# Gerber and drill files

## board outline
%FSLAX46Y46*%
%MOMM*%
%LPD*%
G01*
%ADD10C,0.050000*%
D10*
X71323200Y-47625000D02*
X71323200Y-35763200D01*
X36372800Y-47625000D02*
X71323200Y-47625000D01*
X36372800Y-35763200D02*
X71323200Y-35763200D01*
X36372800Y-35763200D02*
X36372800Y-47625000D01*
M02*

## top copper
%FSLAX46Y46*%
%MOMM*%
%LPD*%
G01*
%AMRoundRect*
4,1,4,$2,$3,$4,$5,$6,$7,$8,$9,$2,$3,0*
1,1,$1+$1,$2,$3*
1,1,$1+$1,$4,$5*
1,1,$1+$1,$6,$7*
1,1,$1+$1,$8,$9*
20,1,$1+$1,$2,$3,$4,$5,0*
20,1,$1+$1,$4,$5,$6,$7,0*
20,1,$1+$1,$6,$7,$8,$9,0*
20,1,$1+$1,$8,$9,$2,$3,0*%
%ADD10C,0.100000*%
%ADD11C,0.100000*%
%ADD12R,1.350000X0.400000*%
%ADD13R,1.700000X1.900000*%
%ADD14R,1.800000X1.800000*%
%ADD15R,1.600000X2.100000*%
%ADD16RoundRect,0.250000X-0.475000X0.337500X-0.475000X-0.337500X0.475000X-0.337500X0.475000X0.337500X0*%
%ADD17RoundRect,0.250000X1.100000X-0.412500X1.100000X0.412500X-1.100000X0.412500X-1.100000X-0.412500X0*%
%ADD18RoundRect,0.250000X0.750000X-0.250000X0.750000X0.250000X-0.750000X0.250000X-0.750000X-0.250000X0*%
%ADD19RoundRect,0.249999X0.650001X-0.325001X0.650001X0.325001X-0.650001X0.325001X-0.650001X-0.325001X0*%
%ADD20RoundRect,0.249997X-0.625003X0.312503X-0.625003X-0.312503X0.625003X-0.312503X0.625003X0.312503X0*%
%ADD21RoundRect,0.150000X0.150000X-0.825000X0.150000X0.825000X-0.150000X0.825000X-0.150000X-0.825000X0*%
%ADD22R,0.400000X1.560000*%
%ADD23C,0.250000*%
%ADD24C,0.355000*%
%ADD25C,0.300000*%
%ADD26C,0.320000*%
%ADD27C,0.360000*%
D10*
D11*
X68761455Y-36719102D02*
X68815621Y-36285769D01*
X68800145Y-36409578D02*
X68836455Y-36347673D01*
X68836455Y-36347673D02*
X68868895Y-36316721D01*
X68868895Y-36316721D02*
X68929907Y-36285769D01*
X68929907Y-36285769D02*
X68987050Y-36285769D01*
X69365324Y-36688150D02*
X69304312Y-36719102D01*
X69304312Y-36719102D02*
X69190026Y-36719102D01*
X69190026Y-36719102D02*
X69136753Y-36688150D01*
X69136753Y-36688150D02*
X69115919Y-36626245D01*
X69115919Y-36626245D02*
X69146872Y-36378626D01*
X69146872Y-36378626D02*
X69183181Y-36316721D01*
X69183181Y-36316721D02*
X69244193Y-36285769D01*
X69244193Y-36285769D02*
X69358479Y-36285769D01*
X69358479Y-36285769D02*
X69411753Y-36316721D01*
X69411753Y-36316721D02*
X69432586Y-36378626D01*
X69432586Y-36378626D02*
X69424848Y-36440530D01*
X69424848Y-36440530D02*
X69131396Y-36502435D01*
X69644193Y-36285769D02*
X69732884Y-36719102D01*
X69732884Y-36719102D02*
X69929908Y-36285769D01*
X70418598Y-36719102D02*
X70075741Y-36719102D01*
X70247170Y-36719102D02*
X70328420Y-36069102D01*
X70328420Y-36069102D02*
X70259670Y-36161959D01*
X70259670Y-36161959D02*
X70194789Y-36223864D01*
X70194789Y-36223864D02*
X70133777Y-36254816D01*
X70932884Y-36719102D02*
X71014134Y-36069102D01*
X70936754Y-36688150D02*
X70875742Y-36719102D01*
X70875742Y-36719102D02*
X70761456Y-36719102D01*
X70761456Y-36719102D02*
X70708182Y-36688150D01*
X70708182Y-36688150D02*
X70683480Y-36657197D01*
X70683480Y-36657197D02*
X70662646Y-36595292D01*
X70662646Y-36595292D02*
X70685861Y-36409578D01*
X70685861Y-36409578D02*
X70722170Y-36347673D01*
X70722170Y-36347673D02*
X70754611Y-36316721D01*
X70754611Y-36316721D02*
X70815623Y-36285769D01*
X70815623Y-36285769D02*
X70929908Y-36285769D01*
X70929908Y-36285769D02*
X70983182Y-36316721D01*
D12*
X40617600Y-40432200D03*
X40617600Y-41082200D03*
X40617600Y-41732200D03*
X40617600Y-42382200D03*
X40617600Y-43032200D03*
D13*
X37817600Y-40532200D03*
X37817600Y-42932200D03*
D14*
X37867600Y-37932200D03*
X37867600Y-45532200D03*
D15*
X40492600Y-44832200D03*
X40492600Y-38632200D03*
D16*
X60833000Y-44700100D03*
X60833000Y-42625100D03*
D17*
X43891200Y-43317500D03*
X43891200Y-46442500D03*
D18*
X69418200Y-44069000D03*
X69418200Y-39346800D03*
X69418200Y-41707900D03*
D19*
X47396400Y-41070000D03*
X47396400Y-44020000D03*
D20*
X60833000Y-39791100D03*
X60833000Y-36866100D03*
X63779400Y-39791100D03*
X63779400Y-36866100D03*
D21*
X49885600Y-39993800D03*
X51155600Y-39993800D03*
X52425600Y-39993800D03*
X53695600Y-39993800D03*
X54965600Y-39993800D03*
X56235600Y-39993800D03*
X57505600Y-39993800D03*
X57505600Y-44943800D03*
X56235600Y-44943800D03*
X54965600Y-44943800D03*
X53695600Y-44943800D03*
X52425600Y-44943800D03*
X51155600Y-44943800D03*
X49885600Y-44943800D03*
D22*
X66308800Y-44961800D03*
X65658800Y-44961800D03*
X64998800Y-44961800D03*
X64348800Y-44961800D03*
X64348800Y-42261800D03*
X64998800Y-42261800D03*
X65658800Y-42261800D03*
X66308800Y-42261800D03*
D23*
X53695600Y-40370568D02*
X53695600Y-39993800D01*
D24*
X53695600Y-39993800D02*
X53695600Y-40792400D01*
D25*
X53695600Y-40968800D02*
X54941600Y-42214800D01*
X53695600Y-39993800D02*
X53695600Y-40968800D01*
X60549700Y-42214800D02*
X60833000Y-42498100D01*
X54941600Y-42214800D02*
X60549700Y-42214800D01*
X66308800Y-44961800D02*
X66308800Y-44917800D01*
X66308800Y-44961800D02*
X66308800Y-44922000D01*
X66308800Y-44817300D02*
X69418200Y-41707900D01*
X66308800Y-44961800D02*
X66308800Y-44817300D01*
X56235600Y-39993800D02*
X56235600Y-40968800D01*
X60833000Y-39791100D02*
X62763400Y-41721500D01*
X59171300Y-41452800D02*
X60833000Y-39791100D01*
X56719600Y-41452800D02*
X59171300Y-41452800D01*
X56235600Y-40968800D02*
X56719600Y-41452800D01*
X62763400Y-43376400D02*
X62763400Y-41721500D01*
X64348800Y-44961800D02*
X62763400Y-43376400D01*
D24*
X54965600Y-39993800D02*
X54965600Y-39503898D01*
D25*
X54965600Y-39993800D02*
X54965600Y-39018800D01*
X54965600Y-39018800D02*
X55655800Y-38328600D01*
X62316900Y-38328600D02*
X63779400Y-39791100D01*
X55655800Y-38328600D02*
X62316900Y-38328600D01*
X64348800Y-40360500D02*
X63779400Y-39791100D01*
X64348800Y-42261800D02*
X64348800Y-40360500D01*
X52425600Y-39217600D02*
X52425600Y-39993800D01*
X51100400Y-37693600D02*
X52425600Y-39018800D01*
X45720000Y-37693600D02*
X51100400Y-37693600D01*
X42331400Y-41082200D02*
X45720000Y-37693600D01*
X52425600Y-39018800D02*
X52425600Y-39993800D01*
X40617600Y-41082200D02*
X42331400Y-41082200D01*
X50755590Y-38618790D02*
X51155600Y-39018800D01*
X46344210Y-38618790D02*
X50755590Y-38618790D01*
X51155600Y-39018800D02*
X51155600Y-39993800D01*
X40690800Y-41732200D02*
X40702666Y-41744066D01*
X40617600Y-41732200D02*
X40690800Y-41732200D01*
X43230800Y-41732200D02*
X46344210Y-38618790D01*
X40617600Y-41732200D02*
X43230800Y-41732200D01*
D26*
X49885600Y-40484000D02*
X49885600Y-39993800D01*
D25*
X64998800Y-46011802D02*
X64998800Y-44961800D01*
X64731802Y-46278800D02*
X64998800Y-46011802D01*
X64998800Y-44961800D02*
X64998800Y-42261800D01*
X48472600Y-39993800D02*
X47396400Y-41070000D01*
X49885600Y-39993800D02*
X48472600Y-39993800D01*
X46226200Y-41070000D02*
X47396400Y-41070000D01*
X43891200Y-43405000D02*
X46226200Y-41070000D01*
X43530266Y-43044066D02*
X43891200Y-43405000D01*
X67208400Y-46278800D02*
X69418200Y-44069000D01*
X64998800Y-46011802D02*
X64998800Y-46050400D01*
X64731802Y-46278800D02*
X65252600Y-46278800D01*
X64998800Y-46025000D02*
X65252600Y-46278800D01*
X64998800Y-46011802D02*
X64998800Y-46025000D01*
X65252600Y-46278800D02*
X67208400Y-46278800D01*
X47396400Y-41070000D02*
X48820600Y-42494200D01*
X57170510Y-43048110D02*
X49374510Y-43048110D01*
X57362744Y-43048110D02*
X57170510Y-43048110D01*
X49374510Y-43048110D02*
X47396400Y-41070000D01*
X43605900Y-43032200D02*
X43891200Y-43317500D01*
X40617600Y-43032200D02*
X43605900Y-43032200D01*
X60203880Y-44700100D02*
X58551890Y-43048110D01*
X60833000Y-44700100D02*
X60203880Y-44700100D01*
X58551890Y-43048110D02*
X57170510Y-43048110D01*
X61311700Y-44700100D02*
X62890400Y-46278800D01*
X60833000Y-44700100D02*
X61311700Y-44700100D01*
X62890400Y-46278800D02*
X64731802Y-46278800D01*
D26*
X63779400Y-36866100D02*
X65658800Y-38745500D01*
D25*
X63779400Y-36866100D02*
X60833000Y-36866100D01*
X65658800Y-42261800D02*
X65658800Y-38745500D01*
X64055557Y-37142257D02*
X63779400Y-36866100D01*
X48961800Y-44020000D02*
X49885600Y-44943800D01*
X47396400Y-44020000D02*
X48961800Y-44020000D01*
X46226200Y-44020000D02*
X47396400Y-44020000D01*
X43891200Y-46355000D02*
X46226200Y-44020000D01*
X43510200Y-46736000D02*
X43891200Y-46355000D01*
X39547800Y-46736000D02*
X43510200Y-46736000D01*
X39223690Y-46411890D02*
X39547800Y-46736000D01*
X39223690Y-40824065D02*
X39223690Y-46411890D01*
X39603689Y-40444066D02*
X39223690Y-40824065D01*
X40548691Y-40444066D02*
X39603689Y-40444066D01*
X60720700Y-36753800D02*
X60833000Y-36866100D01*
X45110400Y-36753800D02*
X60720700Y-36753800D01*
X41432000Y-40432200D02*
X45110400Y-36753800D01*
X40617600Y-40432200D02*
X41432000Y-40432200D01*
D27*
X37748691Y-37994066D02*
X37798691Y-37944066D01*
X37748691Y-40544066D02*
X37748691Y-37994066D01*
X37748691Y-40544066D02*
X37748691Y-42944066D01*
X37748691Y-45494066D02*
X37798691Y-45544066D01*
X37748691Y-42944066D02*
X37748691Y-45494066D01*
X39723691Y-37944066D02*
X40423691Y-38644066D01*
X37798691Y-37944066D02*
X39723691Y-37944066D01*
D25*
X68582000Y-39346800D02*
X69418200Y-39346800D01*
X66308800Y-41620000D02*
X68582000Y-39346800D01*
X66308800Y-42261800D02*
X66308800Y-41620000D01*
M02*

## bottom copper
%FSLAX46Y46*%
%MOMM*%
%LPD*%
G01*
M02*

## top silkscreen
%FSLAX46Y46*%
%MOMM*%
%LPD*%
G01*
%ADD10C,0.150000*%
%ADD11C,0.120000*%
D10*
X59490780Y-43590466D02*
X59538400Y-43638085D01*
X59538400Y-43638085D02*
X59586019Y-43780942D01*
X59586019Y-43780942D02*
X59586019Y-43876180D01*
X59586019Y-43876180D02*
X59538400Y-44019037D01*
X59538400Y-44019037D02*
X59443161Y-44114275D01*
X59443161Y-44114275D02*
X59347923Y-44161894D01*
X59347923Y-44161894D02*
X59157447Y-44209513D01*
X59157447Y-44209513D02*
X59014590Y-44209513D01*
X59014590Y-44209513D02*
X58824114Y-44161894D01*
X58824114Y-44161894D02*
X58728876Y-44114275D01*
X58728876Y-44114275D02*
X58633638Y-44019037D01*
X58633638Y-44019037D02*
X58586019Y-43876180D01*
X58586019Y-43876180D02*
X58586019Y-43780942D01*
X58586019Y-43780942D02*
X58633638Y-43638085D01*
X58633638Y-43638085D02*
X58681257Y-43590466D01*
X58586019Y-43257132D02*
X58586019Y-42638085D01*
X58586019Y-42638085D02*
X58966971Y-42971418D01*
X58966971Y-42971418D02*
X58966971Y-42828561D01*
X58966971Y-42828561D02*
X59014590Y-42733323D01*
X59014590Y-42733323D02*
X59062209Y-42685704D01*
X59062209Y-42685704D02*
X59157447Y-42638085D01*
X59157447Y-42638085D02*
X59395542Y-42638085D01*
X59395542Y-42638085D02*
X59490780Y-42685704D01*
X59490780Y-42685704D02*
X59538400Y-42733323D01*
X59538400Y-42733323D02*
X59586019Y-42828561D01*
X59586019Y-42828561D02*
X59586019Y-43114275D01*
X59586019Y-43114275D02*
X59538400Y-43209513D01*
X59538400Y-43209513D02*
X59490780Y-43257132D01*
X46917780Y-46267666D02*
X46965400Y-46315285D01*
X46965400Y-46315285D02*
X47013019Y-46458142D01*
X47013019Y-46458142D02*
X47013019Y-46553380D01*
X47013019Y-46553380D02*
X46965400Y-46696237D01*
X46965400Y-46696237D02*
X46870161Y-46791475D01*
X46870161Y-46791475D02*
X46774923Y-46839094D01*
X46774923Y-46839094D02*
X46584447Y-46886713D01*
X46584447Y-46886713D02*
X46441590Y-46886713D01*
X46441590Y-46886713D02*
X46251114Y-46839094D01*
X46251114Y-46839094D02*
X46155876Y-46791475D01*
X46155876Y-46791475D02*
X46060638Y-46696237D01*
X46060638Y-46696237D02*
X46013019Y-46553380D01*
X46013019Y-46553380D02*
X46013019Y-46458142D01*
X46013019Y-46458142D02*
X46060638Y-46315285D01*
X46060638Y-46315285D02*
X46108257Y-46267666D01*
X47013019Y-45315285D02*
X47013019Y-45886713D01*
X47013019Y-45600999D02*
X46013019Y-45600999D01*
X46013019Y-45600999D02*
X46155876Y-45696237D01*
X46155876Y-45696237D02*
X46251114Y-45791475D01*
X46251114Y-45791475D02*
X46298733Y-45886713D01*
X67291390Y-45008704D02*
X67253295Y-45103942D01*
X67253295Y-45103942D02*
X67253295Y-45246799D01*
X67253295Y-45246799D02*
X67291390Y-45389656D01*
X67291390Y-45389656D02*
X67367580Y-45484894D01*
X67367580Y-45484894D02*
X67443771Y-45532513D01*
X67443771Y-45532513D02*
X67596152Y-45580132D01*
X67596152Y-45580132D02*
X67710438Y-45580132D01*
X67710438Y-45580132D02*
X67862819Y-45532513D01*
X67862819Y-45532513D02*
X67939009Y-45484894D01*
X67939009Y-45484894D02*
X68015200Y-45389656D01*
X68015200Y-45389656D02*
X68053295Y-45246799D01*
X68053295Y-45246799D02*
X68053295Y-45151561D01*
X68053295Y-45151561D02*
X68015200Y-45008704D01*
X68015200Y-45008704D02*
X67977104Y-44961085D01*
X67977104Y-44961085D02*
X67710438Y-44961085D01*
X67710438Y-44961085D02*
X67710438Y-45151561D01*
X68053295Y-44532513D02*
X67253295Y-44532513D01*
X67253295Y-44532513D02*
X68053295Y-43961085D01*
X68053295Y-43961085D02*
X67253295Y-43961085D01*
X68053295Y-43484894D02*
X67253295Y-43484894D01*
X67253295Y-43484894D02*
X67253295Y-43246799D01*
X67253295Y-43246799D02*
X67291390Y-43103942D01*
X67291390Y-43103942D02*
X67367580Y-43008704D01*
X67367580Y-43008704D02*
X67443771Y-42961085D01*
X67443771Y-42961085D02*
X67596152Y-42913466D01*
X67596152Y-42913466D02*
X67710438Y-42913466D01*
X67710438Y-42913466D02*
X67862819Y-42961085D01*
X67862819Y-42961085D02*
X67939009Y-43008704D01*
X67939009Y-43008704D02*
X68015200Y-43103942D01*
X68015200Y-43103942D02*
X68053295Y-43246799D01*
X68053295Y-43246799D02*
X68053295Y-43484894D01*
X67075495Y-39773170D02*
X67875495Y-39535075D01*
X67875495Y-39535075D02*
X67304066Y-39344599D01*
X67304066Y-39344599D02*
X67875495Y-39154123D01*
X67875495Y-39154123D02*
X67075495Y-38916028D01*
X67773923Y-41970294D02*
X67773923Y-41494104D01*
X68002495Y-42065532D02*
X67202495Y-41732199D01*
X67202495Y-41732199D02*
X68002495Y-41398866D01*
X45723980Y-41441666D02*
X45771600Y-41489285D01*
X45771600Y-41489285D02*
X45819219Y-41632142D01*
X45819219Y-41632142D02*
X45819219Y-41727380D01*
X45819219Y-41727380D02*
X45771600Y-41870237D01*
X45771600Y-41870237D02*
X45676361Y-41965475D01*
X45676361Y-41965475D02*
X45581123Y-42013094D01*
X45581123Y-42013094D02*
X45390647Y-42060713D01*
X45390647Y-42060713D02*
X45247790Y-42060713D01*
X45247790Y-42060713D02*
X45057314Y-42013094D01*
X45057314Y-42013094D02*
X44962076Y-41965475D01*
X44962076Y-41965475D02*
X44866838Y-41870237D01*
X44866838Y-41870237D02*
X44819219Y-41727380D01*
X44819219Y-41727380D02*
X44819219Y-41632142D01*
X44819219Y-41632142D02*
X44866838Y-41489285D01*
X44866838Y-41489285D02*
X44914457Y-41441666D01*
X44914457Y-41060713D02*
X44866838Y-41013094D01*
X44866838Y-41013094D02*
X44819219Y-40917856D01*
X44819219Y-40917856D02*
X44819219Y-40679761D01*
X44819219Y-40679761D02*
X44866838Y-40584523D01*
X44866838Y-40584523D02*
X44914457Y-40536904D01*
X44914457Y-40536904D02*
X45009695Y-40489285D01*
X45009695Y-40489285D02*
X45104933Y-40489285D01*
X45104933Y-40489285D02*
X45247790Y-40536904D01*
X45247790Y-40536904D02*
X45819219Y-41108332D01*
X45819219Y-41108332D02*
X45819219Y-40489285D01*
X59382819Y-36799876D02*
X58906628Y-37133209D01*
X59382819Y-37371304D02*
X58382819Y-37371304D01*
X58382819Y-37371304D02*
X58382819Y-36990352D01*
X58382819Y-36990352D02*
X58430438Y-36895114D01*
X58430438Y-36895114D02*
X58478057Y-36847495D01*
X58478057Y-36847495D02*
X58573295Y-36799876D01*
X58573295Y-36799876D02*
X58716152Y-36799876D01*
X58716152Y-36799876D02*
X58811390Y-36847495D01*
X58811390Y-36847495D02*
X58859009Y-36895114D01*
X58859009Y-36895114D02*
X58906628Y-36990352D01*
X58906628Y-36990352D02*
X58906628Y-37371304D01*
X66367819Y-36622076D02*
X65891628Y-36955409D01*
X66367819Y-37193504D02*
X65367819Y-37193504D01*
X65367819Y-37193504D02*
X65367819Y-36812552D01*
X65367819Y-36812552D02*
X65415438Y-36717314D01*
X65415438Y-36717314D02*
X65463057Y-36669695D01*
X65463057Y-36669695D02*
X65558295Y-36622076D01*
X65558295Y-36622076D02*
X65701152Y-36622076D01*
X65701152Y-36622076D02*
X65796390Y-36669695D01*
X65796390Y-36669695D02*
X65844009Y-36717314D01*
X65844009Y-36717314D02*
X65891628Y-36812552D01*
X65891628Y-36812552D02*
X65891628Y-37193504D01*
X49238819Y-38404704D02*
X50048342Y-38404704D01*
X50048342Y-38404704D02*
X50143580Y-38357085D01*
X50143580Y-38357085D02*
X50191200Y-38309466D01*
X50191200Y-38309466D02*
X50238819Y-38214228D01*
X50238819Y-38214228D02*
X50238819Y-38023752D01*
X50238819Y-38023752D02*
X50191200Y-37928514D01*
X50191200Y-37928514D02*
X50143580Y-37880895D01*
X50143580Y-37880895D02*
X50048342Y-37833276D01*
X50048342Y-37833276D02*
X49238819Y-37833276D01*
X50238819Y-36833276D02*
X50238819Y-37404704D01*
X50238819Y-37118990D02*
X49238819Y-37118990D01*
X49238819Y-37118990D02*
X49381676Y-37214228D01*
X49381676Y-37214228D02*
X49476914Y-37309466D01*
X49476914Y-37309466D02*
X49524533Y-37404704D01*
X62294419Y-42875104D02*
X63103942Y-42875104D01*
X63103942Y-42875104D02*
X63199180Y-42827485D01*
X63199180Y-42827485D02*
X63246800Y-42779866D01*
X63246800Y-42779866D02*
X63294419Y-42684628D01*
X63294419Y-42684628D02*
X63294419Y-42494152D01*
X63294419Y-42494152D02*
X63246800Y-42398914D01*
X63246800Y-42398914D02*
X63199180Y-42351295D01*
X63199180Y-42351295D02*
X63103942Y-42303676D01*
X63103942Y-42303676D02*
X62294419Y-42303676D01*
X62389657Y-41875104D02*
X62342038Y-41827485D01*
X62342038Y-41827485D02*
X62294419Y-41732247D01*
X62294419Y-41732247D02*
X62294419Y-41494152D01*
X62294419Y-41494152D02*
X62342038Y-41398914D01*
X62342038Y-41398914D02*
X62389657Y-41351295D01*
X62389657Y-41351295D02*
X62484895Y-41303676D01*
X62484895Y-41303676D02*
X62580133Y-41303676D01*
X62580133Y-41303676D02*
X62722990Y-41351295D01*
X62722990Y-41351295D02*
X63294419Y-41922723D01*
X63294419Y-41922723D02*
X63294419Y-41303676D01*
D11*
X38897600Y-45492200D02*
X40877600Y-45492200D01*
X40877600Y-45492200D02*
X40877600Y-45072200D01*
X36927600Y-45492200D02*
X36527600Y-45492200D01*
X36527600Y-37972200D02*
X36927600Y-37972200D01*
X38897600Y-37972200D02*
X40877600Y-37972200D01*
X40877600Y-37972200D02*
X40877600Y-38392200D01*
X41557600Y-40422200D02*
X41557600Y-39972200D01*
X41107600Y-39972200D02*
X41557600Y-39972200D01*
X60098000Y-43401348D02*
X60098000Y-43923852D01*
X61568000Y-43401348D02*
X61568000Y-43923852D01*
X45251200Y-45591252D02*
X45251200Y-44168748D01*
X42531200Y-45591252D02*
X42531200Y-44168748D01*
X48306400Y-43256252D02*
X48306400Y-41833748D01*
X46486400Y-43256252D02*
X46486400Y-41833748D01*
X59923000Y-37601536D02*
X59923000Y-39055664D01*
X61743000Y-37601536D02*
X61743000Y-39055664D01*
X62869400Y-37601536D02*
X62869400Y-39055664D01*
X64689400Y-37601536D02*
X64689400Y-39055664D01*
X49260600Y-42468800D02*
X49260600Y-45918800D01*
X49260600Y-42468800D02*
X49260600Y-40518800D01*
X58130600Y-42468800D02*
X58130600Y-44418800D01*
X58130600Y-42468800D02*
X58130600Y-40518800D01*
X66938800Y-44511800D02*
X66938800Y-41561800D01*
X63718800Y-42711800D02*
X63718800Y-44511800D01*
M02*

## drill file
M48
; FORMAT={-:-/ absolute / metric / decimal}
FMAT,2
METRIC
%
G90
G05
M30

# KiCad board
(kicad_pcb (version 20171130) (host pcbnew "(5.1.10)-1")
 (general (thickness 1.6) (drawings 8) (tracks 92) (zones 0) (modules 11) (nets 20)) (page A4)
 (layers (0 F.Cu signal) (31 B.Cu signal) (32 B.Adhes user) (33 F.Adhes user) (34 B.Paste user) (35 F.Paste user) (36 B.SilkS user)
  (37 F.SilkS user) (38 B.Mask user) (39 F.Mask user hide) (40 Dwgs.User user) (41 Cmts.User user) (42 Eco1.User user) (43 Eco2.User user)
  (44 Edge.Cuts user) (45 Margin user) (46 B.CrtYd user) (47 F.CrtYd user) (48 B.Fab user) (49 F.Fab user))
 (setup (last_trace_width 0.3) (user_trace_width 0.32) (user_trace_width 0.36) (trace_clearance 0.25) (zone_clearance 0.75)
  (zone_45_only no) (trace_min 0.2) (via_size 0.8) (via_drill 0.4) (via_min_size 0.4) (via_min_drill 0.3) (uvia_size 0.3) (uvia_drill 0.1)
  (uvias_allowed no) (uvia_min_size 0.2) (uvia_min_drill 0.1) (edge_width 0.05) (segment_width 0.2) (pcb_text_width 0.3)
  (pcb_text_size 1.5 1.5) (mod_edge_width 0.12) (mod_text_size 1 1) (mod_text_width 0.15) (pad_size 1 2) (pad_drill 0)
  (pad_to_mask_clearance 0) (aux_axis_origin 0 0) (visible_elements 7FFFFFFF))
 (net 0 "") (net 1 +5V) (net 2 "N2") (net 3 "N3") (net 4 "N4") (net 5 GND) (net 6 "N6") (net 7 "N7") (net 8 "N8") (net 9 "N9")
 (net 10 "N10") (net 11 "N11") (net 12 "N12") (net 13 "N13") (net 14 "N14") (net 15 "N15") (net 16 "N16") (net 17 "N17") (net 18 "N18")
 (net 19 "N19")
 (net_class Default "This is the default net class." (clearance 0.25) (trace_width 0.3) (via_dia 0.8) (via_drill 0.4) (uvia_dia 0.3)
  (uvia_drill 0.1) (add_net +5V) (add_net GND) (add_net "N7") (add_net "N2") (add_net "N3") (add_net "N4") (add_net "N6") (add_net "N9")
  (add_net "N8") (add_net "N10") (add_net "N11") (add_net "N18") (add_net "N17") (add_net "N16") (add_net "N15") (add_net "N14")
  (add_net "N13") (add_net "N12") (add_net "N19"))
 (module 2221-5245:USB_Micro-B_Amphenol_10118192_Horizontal (layer F.Cu) (at 39.2176 41.7322 270)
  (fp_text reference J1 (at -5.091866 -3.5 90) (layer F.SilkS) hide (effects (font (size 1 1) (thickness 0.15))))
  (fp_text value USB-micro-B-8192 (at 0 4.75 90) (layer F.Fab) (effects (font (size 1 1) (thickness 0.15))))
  (fp_line (start 3.76 0.32) (end 3.76 -1.66) (layer F.SilkS) (width 0.12))
  (fp_line (start 3.76 -1.66) (end 3.34 -1.66) (layer F.SilkS) (width 0.12))
  (fp_line (start 3.76 2.29) (end 3.76 2.69) (layer F.SilkS) (width 0.12))
  (fp_line (start -3.76 2.69) (end -3.76 2.29) (layer F.SilkS) (width 0.12))
  (fp_line (start -3.76 0.32) (end -3.76 -1.66) (layer F.SilkS) (width 0.12))
  (fp_line (start -3.76 -1.66) (end -3.34 -1.66) (layer F.SilkS) (width 0.12))
  (fp_line (start -1.31 -2.34) (end -1.76 -2.34) (layer F.SilkS) (width 0.12))
  (fp_line (start -1.76 -1.89) (end -1.76 -2.34) (layer F.SilkS) (width 0.12))
  (pad 1 smd rect (at -1.3 -1.4 270) (size 0.4 1.35) (layers F.Cu F.Paste F.Mask) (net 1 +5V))
  (pad 2 smd rect (at -0.65 -1.4 270) (size 0.4 1.35) (layers F.Cu F.Paste F.Mask) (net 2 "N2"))
  (pad 3 smd rect (at 0 -1.4 270) (size 0.4 1.35) (layers F.Cu F.Paste F.Mask) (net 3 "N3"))
  (pad 4 smd rect (at 0.65 -1.4 270) (size 0.4 1.35) (layers F.Cu F.Paste) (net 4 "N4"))
  (pad 5 smd rect (at 1.3 -1.4 270) (size 0.4 1.35) (layers F.Cu F.Paste F.Mask) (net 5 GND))
  (pad 6 smd rect (at -1.2 1.4 270) (size 1.9 1.7) (layers F.Cu F.Paste F.Mask) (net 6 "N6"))
  (pad 6 smd rect (at 1.2 1.4 270) (size 1.9 1.7) (layers F.Cu F.Paste F.Mask) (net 6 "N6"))
  (pad 6 smd rect (at -3.8 1.35 270) (size 1.8 1.8) (layers F.Cu F.Paste F.Mask) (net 6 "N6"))
  (pad 6 smd rect (at 3.8 1.35 270) (size 1.8 1.8) (layers F.Cu F.Paste F.Mask) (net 6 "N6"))
  (pad 6 smd rect (at 3.1 -1.275 270) (size 2.1 1.6) (layers F.Cu F.Paste F.Mask) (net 6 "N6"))
  (pad 6 smd rect (at -3.1 -1.275 270) (size 2.1 1.6) (layers F.Cu F.Paste F.Mask) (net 6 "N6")))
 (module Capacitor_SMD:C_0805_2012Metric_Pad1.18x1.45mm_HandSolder (layer F.Cu) (at 60.833 43.6626 270)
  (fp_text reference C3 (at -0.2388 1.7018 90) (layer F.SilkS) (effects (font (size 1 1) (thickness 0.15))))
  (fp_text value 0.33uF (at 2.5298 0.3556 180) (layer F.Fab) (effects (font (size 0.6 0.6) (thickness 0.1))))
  (fp_line (start -0.261252 0.735) (end 0.261252 0.735) (layer F.SilkS) (width 0.12))
  (fp_line (start -0.261252 -0.735) (end 0.261252 -0.735) (layer F.SilkS) (width 0.12))
  (pad 2 smd roundrect (at 1.0375 0 270) (size 1.175 1.45) (layers F.Cu F.Paste F.Mask) (roundrect_rratio 0.212766) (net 5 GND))
  (pad 1 smd roundrect (at -1.0375 0 270) (size 1.175 1.45) (layers F.Cu F.Paste F.Mask) (roundrect_rratio 0.212766) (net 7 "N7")))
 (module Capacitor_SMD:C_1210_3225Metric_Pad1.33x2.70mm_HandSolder (layer F.Cu) (at 43.8912 44.88 90)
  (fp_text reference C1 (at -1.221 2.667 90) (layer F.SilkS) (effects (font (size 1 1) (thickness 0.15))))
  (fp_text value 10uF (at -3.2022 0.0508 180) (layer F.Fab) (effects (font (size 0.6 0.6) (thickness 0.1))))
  (fp_line (start -0.711252 1.36) (end 0.711252 1.36) (layer F.SilkS) (width 0.12))
  (fp_line (start -0.711252 -1.36) (end 0.711252 -1.36) (layer F.SilkS) (width 0.12))
  (pad 2 smd roundrect (at 1.5625 0 90) (size 1.325 2.7) (layers F.Cu F.Paste F.Mask) (roundrect_rratio 0.188679) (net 5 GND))
  (pad 1 smd roundrect (at -1.5625 0 90) (size 1.325 2.7) (layers F.Cu F.Paste F.Mask) (roundrect_rratio 0.188679) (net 1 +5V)))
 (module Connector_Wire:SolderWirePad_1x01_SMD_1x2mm (layer F.Cu) (at 69.4182 44.069 90)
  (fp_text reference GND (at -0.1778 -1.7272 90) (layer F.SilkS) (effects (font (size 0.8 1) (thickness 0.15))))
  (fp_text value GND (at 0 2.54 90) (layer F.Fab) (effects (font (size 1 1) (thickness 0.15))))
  (pad 1 smd roundrect (at 0 0 90) (size 1 2) (layers F.Cu F.Mask) (roundrect_rratio 0.25) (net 5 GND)))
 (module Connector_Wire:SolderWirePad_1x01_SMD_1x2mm (layer F.Cu) (at 69.4182 39.3468 90)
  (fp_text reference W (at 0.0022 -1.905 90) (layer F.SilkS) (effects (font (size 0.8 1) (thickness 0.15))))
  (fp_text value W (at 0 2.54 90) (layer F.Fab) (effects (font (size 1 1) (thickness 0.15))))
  (pad 1 smd roundrect (at 0 0 90) (size 1 2) (layers F.Cu F.Mask) (roundrect_rratio 0.25) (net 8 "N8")))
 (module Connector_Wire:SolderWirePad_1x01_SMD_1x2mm (layer F.Cu) (at 69.4182 41.7068 90)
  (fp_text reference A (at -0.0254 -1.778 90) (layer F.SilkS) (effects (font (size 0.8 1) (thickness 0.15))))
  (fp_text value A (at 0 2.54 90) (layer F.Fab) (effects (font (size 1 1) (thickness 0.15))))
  (pad 1 smd roundrect (at -0.0011 0 90) (size 1 2) (layers F.Cu F.Mask) (roundrect_rratio 0.25) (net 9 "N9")))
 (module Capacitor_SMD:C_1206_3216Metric (layer F.Cu) (at 47.3964 42.545 90)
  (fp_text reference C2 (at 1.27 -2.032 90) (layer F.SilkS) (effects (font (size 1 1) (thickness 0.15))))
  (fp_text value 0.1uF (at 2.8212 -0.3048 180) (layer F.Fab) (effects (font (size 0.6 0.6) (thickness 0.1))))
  (fp_line (start -0.711252 0.91) (end 0.711252 0.91) (layer F.SilkS) (width 0.12))
  (fp_line (start -0.711252 -0.91) (end 0.711252 -0.91) (layer F.SilkS) (width 0.12))
  (pad 2 smd roundrect (at 1.475 0 90) (size 1.15 1.8) (layers F.Cu F.Paste F.Mask) (roundrect_rratio 0.2173904347826087) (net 5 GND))
  (pad 1 smd roundrect (at -1.475 0 90) (size 1.15 1.8) (layers F.Cu F.Paste F.Mask) (roundrect_rratio 0.2173904347826087) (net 1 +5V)))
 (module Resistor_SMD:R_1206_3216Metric (layer F.Cu) (at 60.833 38.3286 270)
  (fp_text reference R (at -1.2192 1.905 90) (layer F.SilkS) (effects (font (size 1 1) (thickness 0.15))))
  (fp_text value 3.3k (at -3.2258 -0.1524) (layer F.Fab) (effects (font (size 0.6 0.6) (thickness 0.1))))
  (fp_line (start -0.727064 0.91) (end 0.727064 0.91) (layer F.SilkS) (width 0.12))
  (fp_line (start -0.727064 -0.91) (end 0.727064 -0.91) (layer F.SilkS) (width 0.12))
  (pad 2 smd roundrect (at 1.4625 0 270) (size 1.125 1.75) (layers F.Cu F.Paste F.Mask) (roundrect_rratio 0.2222195555555556) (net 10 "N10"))
  (pad 1 smd roundrect (at -1.4625 0 270) (size 1.125 1.75) (layers F.Cu F.Paste F.Mask) (roundrect_rratio 0.2222195555555556) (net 1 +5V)))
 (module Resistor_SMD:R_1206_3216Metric (layer F.Cu) (at 63.7794 38.3286 270)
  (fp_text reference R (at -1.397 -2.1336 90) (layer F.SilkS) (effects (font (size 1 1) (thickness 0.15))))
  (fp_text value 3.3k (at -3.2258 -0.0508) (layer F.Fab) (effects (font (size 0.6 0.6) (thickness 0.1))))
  (fp_line (start -0.727064 0.91) (end 0.727064 0.91) (layer F.SilkS) (width 0.12))
  (fp_line (start -0.727064 -0.91) (end 0.727064 -0.91) (layer F.SilkS) (width 0.12))
  (pad 2 smd roundrect (at 1.4625 0 270) (size 1.125 1.75) (layers F.Cu F.Paste F.Mask) (roundrect_rratio 0.2222195555555556) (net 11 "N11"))
  (pad 1 smd roundrect (at -1.4625 0 270) (size 1.125 1.75) (layers F.Cu F.Paste F.Mask) (roundrect_rratio 0.2222195555555556) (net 1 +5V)))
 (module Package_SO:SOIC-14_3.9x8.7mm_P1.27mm (layer F.Cu) (at 53.6956 42.4688 90)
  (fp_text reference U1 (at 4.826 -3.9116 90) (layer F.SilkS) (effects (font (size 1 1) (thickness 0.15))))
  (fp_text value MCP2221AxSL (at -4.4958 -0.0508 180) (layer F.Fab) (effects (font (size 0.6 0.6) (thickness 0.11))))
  (fp_line (start 0 -4.435) (end -3.45 -4.435) (layer F.SilkS) (width 0.12))
  (fp_line (start 0 -4.435) (end 1.95 -4.435) (layer F.SilkS) (width 0.12))
  (fp_line (start 0 4.435) (end -1.95 4.435) (layer F.SilkS) (width 0.12))
  (fp_line (start 0 4.435) (end 1.95 4.435) (layer F.SilkS) (width 0.12))
  (pad 14 smd roundrect (at 2.475 -3.81 90) (size 1.95 0.6) (layers F.Cu F.Paste F.Mask) (roundrect_rratio 0.25) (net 5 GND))
  (pad 13 smd roundrect (at 2.475 -2.54 90) (size 1.95 0.6) (layers F.Cu F.Paste F.Mask) (roundrect_rratio 0.25) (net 3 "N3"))
  (pad 12 smd roundrect (at 2.475 -1.27 90) (size 1.95 0.6) (layers F.Cu F.Paste F.Mask) (roundrect_rratio 0.25) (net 2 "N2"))
  (pad 11 smd roundrect (at 2.475 0 90) (size 1.95 0.6) (layers F.Cu F.Paste F.Mask) (roundrect_rratio 0.25) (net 7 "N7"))
  (pad 10 smd roundrect (at 2.475 1.27 90) (size 1.95 0.6) (layers F.Cu F.Paste F.Mask) (roundrect_rratio 0.25) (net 11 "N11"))
  (pad 9 smd roundrect (at 2.475 2.54 90) (size 1.95 0.6) (layers F.Cu F.Paste F.Mask) (roundrect_rratio 0.25) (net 10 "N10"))
  (pad 8 smd roundrect (at 2.475 3.81 90) (size 1.95 0.6) (layers F.Cu F.Paste F.Mask) (roundrect_rratio 0.25) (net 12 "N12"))
  (pad 7 smd roundrect (at -2.475 3.81 90) (size 1.95 0.6) (layers F.Cu F.Paste F.Mask) (roundrect_rratio 0.25) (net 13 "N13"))
  (pad 6 smd roundrect (at -2.475 2.54 90) (size 1.95 0.6) (layers F.Cu F.Paste F.Mask) (roundrect_rratio 0.25) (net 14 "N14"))
  (pad 5 smd roundrect (at -2.475 1.27 90) (size 1.95 0.6) (layers F.Cu F.Paste F.Mask) (roundrect_rratio 0.25) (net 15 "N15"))
  (pad 4 smd roundrect (at -2.475 0 90) (size 1.95 0.6) (layers F.Cu F.Paste F.Mask) (roundrect_rratio 0.25) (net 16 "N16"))
  (pad 3 smd roundrect (at -2.475 -1.27 90) (size 1.95 0.6) (layers F.Cu F.Paste F.Mask) (roundrect_rratio 0.25) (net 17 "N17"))
  (pad 2 smd roundrect (at -2.475 -2.54 90) (size 1.95 0.6) (layers F.Cu F.Paste F.Mask) (roundrect_rratio 0.25) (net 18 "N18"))
  (pad 1 smd roundrect (at -2.475 -3.81 90) (size 1.95 0.6) (layers F.Cu F.Paste F.Mask) (roundrect_rratio 0.25) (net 1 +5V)))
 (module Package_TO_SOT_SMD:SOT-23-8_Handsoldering (layer F.Cu) (at 65.3288 43.6118 270)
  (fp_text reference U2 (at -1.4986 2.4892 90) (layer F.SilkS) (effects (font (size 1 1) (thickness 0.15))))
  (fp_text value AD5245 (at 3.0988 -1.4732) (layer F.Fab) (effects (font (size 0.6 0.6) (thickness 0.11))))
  (fp_line (start 0.9 -1.61) (end -2.05 -1.61) (layer F.SilkS) (width 0.12))
  (fp_line (start -0.9 1.61) (end 0.9 1.61) (layer F.SilkS) (width 0.12))
  (pad 8 smd rect (at 1.35 -0.98 270) (size 1.56 0.4) (layers F.Cu F.Paste F.Mask) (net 9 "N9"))
  (pad 7 smd rect (at 1.35 -0.33 270) (size 1.56 0.4) (layers F.Cu F.Paste F.Mask) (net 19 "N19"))
  (pad 6 smd rect (at 1.35 0.33 270) (size 1.56 0.4) (layers F.Cu F.Paste F.Mask) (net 5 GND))
  (pad 5 smd rect (at 1.35 0.98 270) (size 1.56 0.4) (layers F.Cu F.Paste F.Mask) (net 10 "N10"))
  (pad 4 smd rect (at -1.35 0.98 270) (size 1.56 0.4) (layers F.Cu F.Paste F.Mask) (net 11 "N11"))
  (pad 3 smd rect (at -1.35 0.33 270) (size 1.56 0.4) (layers F.Cu F.Paste F.Mask) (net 5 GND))
  (pad 2 smd rect (at -1.35 -0.33 270) (size 1.56 0.4) (layers F.Cu F.Paste F.Mask) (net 1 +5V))
  (pad 1 smd rect (at -1.35 -0.98 270) (size 1.56 0.4) (layers F.Cu F.Paste F.Mask) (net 8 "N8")))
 (gr_line (start 71.3232 47.625) (end 71.3232 35.7632) (layer Edge.Cuts) (width 0.05))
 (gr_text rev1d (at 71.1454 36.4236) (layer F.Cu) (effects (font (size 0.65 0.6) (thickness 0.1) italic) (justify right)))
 (gr_line (start 36.3728 47.625) (end 71.3232 47.625) (layer Edge.Cuts) (width 0.05))
 (gr_line (start 36.3728 35.7632) (end 71.3232 35.7632) (layer Edge.Cuts) (width 0.05))
 (gr_line (start 36.3728 35.7632) (end 36.3728 47.625) (layer Edge.Cuts) (width 0.05))
 (segment (start 53.6956 40.370568) (end 53.6956 39.9938) (width 0.25) (layer F.Cu) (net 7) (status 30))
 (segment (start 53.6956 39.9938) (end 53.6956 40.7924) (width 0.355) (layer F.Cu) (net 7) (status 30))
 (segment (start 53.6956 40.9688) (end 54.9416 42.2148) (width 0.3) (layer F.Cu) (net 7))
 (segment (start 53.6956 39.9938) (end 53.6956 40.9688) (width 0.3) (layer F.Cu) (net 7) (status 10))
 (segment (start 60.5497 42.2148) (end 60.833 42.4981) (width 0.3) (layer F.Cu) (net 7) (status 30))
 (segment (start 54.9416 42.2148) (end 60.5497 42.2148) (width 0.3) (layer F.Cu) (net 7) (status 20))
 (segment (start 66.3088 44.9618) (end 66.3088 44.9178) (width 0.3) (layer F.Cu) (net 9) (status 30))
 (segment (start 66.3088 44.9618) (end 66.3088 44.922) (width 0.3) (layer F.Cu) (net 9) (status 30))
 (segment (start 66.3088 44.8173) (end 69.4182 41.7079) (width 0.3) (layer F.Cu) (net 9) (status 30))
 (segment (start 66.3088 44.9618) (end 66.3088 44.8173) (width 0.3) (layer F.Cu) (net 9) (status 30))
 (segment (start 56.2356 39.9938) (end 56.2356 40.9688) (width 0.3) (layer F.Cu) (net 10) (status 10))
 (segment (start 60.833 39.7911) (end 62.7634 41.7215) (width 0.3) (layer F.Cu) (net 10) (status 10))
 (segment (start 59.1713 41.4528) (end 60.833 39.7911) (width 0.3) (layer F.Cu) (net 10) (status 20))
 (segment (start 56.7196 41.4528) (end 59.1713 41.4528) (width 0.3) (layer F.Cu) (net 10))
 (segment (start 56.2356 40.9688) (end 56.7196 41.4528) (width 0.3) (layer F.Cu) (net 10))
 (segment (start 62.7634 43.3764) (end 62.7634 41.7215) (width 0.3) (layer F.Cu) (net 10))
 (segment (start 64.3488 44.9618) (end 62.7634 43.3764) (width 0.3) (layer F.Cu) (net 10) (status 10))
 (segment (start 54.9656 39.9938) (end 54.9656 39.503898) (width 0.355) (layer F.Cu) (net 11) (status 30))
 (segment (start 54.9656 39.9938) (end 54.9656 39.0188) (width 0.3) (layer F.Cu) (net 11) (status 30))
 (segment (start 54.9656 39.0188) (end 55.6558 38.3286) (width 0.3) (layer F.Cu) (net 11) (status 10))
 (segment (start 62.3169 38.3286) (end 63.7794 39.7911) (width 0.3) (layer F.Cu) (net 11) (status 20))
 (segment (start 55.6558 38.3286) (end 62.3169 38.3286) (width 0.3) (layer F.Cu) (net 11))
 (segment (start 64.3488 40.3605) (end 63.7794 39.7911) (width 0.3) (layer F.Cu) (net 11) (status 20))
 (segment (start 64.3488 42.2618) (end 64.3488 40.3605) (width 0.3) (layer F.Cu) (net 11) (status 10))
 (segment (start 52.4256 39.2176) (end 52.4256 39.9938) (width 0.3) (layer F.Cu) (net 2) (status 30))
 (segment (start 51.1004 37.6936) (end 52.4256 39.0188) (width 0.3) (layer F.Cu) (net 2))
 (segment (start 45.72 37.6936) (end 51.1004 37.6936) (width 0.3) (layer F.Cu) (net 2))
 (segment (start 42.3314 41.0822) (end 45.72 37.6936) (width 0.3) (layer F.Cu) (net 2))
 (segment (start 52.4256 39.0188) (end 52.4256 39.9938) (width 0.3) (layer F.Cu) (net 2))
 (segment (start 40.6176 41.0822) (end 42.3314 41.0822) (width 0.3) (layer F.Cu) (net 2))
 (segment (start 50.75559 38.61879) (end 51.1556 39.0188) (width 0.3) (layer F.Cu) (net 3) (status 20))
 (segment (start 46.34421 38.61879) (end 50.75559 38.61879) (width 0.3) (layer F.Cu) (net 3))
 (segment (start 51.1556 39.0188) (end 51.1556 39.9938) (width 0.3) (layer F.Cu) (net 3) (status 30))
 (segment (start 40.6908 41.7322) (end 40.702666 41.744066) (width 0.3) (layer F.Cu) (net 3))
 (segment (start 40.6176 41.7322) (end 40.6908 41.7322) (width 0.3) (layer F.Cu) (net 3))
 (segment (start 43.2308 41.7322) (end 46.34421 38.61879) (width 0.3) (layer F.Cu) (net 3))
 (segment (start 40.6176 41.7322) (end 43.2308 41.7322) (width 0.3) (layer F.Cu) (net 3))
 (segment (start 49.8856 40.484) (end 49.8856 39.9938) (width 0.32) (layer F.Cu) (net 5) (status 30))
 (segment (start 64.9988 46.011802) (end 64.9988 44.9618) (width 0.3) (layer F.Cu) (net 5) (status 20))
 (segment (start 64.731802 46.2788) (end 64.9988 46.011802) (width 0.3) (layer F.Cu) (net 5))
 (segment (start 64.9988 44.9618) (end 64.9988 42.2618) (width 0.3) (layer F.Cu) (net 5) (status 30))
 (segment (start 48.4726 39.9938) (end 47.3964 41.07) (width 0.3) (layer F.Cu) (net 5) (status 20))
 (segment (start 49.8856 39.9938) (end 48.4726 39.9938) (width 0.3) (layer F.Cu) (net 5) (status 10))
 (segment (start 46.2262 41.07) (end 47.3964 41.07) (width 0.3) (layer F.Cu) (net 5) (status 20))
 (segment (start 43.8912 43.405) (end 46.2262 41.07) (width 0.3) (layer F.Cu) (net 5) (status 10))
 (segment (start 43.530266 43.044066) (end 43.8912 43.405) (width 0.3) (layer F.Cu) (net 5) (status 30))
 (segment (start 67.2084 46.2788) (end 69.4182 44.069) (width 0.3) (layer F.Cu) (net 5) (status 20))
 (segment (start 64.9988 46.011802) (end 64.9988 46.0504) (width 0.3) (layer F.Cu) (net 5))
 (segment (start 64.731802 46.2788) (end 65.2526 46.2788) (width 0.3) (layer F.Cu) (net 5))
 (segment (start 64.9988 46.025) (end 65.2526 46.2788) (width 0.3) (layer F.Cu) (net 5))
 (segment (start 64.9988 46.011802) (end 64.9988 46.025) (width 0.3) (layer F.Cu) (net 5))
 (segment (start 65.2526 46.2788) (end 67.2084 46.2788) (width 0.3) (layer F.Cu) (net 5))
 (segment (start 47.3964 41.07) (end 48.8206 42.4942) (width 0.3) (layer F.Cu) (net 5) (status 10))
 (segment (start 57.17051 43.04811) (end 49.37451 43.04811) (width 0.3) (layer F.Cu) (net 5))
 (segment (start 57.362744 43.04811) (end 57.17051 43.04811) (width 0.3) (layer F.Cu) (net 5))
 (segment (start 49.37451 43.04811) (end 47.3964 41.07) (width 0.3) (layer F.Cu) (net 5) (status 20))
 (segment (start 43.6059 43.0322) (end 43.8912 43.3175) (width 0.3) (layer F.Cu) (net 5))
 (segment (start 40.6176 43.0322) (end 43.6059 43.0322) (width 0.3) (layer F.Cu) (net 5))
 (segment (start 60.20388 44.7001) (end 58.55189 43.04811) (width 0.3) (layer F.Cu) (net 5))
 (segment (start 60.833 44.7001) (end 60.20388 44.7001) (width 0.3) (layer F.Cu) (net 5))
 (segment (start 58.55189 43.04811) (end 57.17051 43.04811) (width 0.3) (layer F.Cu) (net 5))
 (segment (start 61.3117 44.7001) (end 62.8904 46.2788) (width 0.3) (layer F.Cu) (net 5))
 (segment (start 60.833 44.7001) (end 61.3117 44.7001) (width 0.3) (layer F.Cu) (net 5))
 (segment (start 62.8904 46.2788) (end 64.731802 46.2788) (width 0.3) (layer F.Cu) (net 5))
 (segment (start 63.7794 36.8661) (end 65.6588 38.7455) (width 0.32) (layer F.Cu) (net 1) (status 10))
 (segment (start 63.7794 36.8661) (end 60.833 36.8661) (width 0.3) (layer F.Cu) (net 1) (status 30))
 (segment (start 65.6588 42.2618) (end 65.6588 38.7455) (width 0.3) (layer F.Cu) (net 1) (status 10))
 (segment (start 64.055557 37.142257) (end 63.7794 36.8661) (width 0.3) (layer F.Cu) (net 1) (status 30))
 (segment (start 48.9618 44.02) (end 49.8856 44.9438) (width 0.3) (layer F.Cu) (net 1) (status 20))
 (segment (start 47.3964 44.02) (end 48.9618 44.02) (width 0.3) (layer F.Cu) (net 1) (status 10))
 (segment (start 46.2262 44.02) (end 47.3964 44.02) (width 0.3) (layer F.Cu) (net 1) (status 20))
 (segment (start 43.8912 46.355) (end 46.2262 44.02) (width 0.3) (layer F.Cu) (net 1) (status 10))
 (segment (start 43.5102 46.736) (end 43.8912 46.355) (width 0.3) (layer F.Cu) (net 1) (status 30))
 (segment (start 39.5478 46.736) (end 43.5102 46.736) (width 0.3) (layer F.Cu) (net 1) (status 20))
 (segment (start 39.22369 46.41189) (end 39.5478 46.736) (width 0.3) (layer F.Cu) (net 1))
 (segment (start 39.22369 40.824065) (end 39.22369 46.41189) (width 0.3) (layer F.Cu) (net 1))
 (segment (start 39.603689 40.444066) (end 39.22369 40.824065) (width 0.3) (layer F.Cu) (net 1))
 (segment (start 40.548691 40.444066) (end 39.603689 40.444066) (width 0.3) (layer F.Cu) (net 1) (status 10))
 (segment (start 60.7207 36.7538) (end 60.833 36.8661) (width 0.3) (layer F.Cu) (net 1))
 (segment (start 45.1104 36.7538) (end 60.7207 36.7538) (width 0.3) (layer F.Cu) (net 1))
 (segment (start 41.432 40.4322) (end 45.1104 36.7538) (width 0.3) (layer F.Cu) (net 1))
 (segment (start 40.6176 40.4322) (end 41.432 40.4322) (width 0.3) (layer F.Cu) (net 1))
 (segment (start 37.748691 37.994066) (end 37.798691 37.944066) (width 0.36) (layer F.Cu) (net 6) (status 30))
 (segment (start 37.748691 40.544066) (end 37.748691 37.994066) (width 0.36) (layer F.Cu) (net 6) (status 30))
 (segment (start 37.748691 40.544066) (end 37.748691 42.944066) (width 0.36) (layer F.Cu) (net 6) (status 30))
 (segment (start 37.748691 45.494066) (end 37.798691 45.544066) (width 0.36) (layer F.Cu) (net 6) (status 30))
 (segment (start 37.748691 42.944066) (end 37.748691 45.494066) (width 0.36) (layer F.Cu) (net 6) (status 30))
 (segment (start 39.723691 37.944066) (end 40.423691 38.644066) (width 0.36) (layer F.Cu) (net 6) (status 30))
 (segment (start 37.798691 37.944066) (end 39.723691 37.944066) (width 0.36) (layer F.Cu) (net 6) (status 30))
 (segment (start 68.582 39.3468) (end 69.4182 39.3468) (width 0.3) (layer F.Cu) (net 8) (status 30))
 (segment (start 66.3088 41.62) (end 68.582 39.3468) (width 0.3) (layer F.Cu) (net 8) (status 30))
 (segment (start 66.3088 42.2618) (end 66.3088 41.62) (width 0.3) (layer F.Cu) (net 8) (status 30)))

